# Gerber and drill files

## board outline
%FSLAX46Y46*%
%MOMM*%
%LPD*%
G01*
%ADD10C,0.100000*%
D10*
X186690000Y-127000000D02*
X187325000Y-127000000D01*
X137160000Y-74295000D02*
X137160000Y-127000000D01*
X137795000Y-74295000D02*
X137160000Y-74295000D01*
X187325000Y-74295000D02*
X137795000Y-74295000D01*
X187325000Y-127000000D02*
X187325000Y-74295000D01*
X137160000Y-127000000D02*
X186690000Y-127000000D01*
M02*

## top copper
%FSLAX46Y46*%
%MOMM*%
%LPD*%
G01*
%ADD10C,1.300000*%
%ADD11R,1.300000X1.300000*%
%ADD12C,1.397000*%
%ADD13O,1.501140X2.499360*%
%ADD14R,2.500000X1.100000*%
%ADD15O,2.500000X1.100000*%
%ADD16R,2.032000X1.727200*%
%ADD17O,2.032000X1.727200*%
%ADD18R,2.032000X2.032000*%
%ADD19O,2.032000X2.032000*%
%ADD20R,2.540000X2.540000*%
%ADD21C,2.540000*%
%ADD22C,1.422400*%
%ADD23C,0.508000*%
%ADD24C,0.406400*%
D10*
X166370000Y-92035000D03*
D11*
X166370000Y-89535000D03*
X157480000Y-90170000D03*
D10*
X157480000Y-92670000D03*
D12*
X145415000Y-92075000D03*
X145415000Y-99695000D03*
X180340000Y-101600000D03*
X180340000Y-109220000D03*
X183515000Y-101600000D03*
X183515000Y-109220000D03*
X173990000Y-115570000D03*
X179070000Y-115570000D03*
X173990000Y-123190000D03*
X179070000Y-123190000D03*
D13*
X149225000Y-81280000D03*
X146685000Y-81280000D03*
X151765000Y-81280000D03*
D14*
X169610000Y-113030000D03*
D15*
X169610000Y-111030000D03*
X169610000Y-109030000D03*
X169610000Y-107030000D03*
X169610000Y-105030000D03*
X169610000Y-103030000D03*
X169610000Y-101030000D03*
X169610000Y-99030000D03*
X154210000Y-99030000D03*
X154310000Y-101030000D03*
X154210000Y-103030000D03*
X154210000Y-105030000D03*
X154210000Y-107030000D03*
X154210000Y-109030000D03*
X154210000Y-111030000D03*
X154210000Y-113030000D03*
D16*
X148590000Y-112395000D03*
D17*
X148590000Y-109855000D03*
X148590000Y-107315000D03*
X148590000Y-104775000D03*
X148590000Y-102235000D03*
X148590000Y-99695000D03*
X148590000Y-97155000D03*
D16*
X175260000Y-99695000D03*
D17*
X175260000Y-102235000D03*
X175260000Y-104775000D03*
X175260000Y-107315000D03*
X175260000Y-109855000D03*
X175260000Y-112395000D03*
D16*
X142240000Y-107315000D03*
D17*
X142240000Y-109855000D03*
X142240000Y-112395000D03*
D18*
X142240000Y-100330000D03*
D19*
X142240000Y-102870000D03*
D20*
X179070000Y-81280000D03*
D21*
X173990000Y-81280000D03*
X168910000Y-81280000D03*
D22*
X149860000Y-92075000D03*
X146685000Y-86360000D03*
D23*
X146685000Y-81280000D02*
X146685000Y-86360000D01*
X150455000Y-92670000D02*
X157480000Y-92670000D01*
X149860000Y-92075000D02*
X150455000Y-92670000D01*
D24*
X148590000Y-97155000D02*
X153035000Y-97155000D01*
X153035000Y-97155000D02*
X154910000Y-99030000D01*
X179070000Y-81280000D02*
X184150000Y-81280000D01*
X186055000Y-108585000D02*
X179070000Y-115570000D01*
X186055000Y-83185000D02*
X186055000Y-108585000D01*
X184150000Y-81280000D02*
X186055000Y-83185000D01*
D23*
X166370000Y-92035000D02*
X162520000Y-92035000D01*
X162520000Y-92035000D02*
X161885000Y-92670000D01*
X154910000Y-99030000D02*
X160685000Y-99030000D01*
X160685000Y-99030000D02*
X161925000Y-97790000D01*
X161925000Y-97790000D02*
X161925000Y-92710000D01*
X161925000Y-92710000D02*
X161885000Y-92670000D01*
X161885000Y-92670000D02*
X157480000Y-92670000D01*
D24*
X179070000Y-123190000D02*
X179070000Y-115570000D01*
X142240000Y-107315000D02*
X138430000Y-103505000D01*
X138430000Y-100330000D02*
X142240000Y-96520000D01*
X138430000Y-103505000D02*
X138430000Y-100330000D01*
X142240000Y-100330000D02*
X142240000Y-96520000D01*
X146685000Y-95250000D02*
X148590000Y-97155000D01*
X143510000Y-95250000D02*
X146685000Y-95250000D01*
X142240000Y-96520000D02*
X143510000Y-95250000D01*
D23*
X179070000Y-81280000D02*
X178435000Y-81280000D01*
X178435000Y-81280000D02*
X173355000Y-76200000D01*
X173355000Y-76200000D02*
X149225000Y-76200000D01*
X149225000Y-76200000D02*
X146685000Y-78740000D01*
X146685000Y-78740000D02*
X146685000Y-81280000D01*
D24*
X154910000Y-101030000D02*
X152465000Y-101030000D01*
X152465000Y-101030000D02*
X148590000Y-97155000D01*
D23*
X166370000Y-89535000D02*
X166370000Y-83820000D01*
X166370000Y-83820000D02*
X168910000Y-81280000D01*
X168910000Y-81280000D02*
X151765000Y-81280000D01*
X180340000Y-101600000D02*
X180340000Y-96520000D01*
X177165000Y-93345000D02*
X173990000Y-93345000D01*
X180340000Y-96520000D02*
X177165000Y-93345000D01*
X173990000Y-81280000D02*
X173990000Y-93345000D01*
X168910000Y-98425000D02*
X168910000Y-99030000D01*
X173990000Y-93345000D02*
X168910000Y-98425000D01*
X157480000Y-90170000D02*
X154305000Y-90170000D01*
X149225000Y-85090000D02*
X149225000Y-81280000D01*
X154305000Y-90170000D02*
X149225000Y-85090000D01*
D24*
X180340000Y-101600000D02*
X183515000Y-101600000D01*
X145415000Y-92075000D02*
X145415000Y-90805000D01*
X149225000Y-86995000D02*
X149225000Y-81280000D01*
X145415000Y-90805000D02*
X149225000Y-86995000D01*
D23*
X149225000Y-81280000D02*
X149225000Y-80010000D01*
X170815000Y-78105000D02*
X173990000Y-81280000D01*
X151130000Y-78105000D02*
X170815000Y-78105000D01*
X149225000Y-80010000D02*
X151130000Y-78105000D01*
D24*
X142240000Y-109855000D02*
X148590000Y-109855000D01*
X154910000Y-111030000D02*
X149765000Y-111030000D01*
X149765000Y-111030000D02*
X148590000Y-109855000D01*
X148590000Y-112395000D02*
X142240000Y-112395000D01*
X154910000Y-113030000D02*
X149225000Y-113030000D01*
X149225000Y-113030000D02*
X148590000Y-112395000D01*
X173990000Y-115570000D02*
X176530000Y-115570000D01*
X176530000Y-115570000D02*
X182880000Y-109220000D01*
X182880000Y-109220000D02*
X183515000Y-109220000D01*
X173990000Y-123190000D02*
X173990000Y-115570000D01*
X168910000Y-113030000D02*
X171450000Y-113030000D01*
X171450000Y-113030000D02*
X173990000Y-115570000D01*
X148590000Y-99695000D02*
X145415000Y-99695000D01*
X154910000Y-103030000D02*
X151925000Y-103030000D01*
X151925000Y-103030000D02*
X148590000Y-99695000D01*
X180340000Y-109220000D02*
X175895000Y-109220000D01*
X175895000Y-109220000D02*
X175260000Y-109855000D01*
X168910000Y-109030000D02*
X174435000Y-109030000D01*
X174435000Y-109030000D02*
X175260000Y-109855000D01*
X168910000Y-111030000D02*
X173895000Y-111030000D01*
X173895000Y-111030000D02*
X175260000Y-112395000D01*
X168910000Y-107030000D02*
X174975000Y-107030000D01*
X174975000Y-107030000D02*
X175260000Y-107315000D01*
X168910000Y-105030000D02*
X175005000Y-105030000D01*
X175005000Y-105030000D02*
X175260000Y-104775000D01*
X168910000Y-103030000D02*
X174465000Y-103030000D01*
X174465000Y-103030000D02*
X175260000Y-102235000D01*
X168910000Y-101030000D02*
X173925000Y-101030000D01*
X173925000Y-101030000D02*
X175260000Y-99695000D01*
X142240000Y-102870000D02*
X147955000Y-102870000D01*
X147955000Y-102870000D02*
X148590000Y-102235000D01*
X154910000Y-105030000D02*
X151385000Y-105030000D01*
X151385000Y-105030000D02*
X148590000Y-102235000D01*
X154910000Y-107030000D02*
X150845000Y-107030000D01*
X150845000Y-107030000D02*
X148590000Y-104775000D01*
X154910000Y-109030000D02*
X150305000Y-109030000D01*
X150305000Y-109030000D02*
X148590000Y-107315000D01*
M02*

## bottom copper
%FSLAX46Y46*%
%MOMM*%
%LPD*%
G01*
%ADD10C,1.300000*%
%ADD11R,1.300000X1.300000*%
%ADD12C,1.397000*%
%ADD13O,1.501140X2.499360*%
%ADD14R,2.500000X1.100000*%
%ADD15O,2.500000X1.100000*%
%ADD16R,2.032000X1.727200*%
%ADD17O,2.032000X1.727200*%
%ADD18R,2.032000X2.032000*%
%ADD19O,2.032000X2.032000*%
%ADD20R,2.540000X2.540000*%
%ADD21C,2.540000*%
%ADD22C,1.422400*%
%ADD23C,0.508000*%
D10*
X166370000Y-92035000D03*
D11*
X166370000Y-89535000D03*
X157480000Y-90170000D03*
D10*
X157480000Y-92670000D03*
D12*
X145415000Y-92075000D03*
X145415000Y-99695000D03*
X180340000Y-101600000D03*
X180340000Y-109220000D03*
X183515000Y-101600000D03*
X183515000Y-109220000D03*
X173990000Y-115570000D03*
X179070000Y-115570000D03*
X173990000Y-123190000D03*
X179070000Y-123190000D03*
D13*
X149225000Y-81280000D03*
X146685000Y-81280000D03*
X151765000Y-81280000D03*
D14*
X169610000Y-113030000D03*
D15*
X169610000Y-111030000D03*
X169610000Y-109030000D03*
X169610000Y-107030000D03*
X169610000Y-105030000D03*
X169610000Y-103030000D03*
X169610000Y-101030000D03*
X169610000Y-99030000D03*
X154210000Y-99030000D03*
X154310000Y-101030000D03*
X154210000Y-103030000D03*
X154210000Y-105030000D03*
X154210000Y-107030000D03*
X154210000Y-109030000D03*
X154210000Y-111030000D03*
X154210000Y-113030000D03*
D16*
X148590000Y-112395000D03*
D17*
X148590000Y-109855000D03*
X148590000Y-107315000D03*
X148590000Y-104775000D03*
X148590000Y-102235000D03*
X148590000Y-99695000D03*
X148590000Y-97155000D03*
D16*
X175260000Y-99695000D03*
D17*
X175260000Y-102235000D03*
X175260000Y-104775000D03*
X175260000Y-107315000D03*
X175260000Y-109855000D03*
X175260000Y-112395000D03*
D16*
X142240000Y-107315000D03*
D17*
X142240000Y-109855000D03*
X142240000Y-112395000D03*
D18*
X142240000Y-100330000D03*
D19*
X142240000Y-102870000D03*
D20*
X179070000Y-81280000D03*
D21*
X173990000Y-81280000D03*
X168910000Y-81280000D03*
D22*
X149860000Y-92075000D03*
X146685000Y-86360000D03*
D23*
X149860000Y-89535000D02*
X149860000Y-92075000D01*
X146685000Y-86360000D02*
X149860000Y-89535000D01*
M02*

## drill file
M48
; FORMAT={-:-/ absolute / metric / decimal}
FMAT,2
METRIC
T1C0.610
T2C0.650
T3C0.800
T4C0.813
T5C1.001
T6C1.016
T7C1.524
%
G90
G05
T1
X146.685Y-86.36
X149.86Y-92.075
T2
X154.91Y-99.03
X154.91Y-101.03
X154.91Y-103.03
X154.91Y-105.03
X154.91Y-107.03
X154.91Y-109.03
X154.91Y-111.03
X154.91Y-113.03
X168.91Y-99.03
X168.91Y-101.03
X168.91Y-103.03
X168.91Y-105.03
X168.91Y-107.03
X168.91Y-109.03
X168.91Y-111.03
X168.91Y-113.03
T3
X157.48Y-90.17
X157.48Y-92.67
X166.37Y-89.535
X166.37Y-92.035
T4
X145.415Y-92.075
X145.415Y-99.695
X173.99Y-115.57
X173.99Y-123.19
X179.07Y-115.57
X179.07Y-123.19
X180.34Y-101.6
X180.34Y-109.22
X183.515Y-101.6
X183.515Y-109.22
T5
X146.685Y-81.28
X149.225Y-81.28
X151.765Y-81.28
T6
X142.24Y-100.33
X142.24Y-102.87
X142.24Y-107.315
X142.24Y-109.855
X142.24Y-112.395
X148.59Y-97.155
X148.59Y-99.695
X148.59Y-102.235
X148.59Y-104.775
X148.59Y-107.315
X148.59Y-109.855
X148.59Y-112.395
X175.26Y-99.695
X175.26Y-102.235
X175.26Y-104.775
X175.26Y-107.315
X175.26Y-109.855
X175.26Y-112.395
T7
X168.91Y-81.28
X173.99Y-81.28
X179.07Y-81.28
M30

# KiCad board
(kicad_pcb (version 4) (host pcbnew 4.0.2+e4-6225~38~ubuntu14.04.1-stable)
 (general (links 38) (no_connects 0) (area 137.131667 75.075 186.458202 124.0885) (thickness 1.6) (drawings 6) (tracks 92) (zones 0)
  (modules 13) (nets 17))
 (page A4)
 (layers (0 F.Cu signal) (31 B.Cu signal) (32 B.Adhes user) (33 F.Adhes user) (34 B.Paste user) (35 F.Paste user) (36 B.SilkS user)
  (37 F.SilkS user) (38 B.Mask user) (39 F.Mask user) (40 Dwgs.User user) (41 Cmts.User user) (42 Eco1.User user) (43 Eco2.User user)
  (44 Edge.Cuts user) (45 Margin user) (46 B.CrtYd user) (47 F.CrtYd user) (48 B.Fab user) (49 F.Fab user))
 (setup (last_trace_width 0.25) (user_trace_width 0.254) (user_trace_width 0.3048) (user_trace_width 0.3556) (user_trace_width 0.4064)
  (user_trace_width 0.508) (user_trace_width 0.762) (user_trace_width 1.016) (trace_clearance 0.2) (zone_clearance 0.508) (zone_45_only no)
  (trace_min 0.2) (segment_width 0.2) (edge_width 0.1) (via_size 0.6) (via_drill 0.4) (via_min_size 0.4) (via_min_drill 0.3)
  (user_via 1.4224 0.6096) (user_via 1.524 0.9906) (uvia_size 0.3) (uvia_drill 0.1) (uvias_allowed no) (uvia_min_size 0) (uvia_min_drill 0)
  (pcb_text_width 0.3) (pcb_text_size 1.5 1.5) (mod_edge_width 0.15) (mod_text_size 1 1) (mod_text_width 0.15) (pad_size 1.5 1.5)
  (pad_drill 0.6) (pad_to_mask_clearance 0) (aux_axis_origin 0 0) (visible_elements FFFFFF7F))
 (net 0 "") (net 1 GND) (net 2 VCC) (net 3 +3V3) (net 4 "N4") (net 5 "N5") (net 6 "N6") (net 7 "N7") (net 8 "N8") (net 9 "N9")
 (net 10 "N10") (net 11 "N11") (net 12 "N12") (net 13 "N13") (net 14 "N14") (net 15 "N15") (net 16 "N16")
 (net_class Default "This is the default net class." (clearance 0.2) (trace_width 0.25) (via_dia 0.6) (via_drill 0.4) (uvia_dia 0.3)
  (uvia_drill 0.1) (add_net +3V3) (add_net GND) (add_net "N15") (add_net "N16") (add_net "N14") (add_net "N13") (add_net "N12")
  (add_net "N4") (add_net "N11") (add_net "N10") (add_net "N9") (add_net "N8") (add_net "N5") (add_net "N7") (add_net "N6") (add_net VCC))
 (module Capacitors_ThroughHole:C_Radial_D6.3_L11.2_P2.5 (layer F.Cu) (at 166.37 89.535 270)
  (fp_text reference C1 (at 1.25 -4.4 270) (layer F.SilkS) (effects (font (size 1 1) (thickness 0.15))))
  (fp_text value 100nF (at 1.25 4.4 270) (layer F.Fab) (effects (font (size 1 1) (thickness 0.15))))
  (pad 2 thru_hole circle (at 2.5 0 270) (size 1.3 1.3) (drill 0.8) (layers *.Cu *.Mask F.SilkS) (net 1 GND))
  (pad 1 thru_hole rect (at 0 0 270) (size 1.3 1.3) (drill 0.8) (layers *.Cu *.Mask F.SilkS) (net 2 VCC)))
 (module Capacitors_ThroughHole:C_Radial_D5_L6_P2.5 (layer F.Cu) (at 157.48 90.17 270)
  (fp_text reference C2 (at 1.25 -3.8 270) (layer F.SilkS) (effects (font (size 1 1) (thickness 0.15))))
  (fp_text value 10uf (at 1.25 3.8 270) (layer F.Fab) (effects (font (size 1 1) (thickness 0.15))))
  (pad 1 thru_hole rect (at 0 0 270) (size 1.3 1.3) (drill 0.8) (layers *.Cu *.Mask F.SilkS) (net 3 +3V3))
  (pad 2 thru_hole circle (at 2.5 0 270) (size 1.3 1.3) (drill 0.8) (layers *.Cu *.Mask F.SilkS) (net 1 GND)))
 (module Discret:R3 (layer F.Cu) (at 145.415 95.885 270)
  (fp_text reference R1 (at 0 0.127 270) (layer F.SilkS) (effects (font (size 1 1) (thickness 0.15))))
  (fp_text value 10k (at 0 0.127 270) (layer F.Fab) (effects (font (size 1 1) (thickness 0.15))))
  (pad 1 thru_hole circle (at -3.81 0 270) (size 1.397 1.397) (drill 0.8128) (layers *.Cu *.Mask F.SilkS) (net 3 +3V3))
  (pad 2 thru_hole circle (at 3.81 0 270) (size 1.397 1.397) (drill 0.8128) (layers *.Cu *.Mask F.SilkS) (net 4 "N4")))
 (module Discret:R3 (layer F.Cu) (at 180.34 105.41 270)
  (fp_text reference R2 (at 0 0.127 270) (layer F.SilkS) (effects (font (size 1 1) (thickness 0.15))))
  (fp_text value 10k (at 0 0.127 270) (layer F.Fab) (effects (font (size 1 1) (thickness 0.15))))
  (pad 1 thru_hole circle (at -3.81 0 270) (size 1.397 1.397) (drill 0.8128) (layers *.Cu *.Mask F.SilkS) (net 3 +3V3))
  (pad 2 thru_hole circle (at 3.81 0 270) (size 1.397 1.397) (drill 0.8128) (layers *.Cu *.Mask F.SilkS) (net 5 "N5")))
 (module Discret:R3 (layer F.Cu) (at 183.515 105.41 270)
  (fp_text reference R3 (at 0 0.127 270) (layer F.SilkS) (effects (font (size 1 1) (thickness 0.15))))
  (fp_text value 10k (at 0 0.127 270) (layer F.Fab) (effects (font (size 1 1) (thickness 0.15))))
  (pad 1 thru_hole circle (at -3.81 0 270) (size 1.397 1.397) (drill 0.8128) (layers *.Cu *.Mask F.SilkS) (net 3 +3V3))
  (pad 2 thru_hole circle (at 3.81 0 270) (size 1.397 1.397) (drill 0.8128) (layers *.Cu *.Mask F.SilkS) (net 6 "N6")))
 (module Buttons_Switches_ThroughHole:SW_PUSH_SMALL (layer F.Cu) (at 176.53 119.38 90)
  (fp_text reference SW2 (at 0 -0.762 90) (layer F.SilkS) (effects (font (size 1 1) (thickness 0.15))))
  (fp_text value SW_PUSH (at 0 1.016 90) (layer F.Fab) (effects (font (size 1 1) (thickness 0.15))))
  (pad 1 thru_hole circle (at 3.81 -2.54 90) (size 1.397 1.397) (drill 0.8128) (layers *.Cu *.Mask F.SilkS) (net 6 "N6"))
  (pad 2 thru_hole circle (at 3.81 2.54 90) (size 1.397 1.397) (drill 0.8128) (layers *.Cu *.Mask F.SilkS) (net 1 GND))
  (pad 1 thru_hole circle (at -3.81 -2.54 90) (size 1.397 1.397) (drill 0.8128) (layers *.Cu *.Mask F.SilkS) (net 6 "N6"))
  (pad 2 thru_hole circle (at -3.81 2.54 90) (size 1.397 1.397) (drill 0.8128) (layers *.Cu *.Mask F.SilkS) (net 1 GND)))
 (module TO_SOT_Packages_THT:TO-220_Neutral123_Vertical (layer F.Cu) (at 149.225 81.28)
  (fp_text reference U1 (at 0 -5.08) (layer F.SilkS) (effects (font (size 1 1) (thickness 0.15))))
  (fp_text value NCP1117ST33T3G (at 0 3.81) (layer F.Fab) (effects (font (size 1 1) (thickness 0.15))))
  (pad 2 thru_hole oval (at 0 0 90) (size 2.49936 1.50114) (drill 1.00076) (layers *.Cu *.Mask F.SilkS) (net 3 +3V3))
  (pad 1 thru_hole oval (at -2.54 0 90) (size 2.49936 1.50114) (drill 1.00076) (layers *.Cu *.Mask F.SilkS) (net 1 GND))
  (pad 3 thru_hole oval (at 2.54 0 90) (size 2.49936 1.50114) (drill 1.00076) (layers *.Cu *.Mask F.SilkS) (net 2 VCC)))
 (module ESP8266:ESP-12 (layer F.Cu) (at 168.91 113.03 180)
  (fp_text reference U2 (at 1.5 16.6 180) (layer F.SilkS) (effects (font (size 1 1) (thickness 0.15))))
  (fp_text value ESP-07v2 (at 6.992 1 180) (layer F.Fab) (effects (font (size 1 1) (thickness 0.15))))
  (pad 1 thru_hole rect (at 0 0 180) (size 2.5 1.1) (drill 0.65 (offset -0.7 0)) (layers *.Cu *.Mask F.SilkS) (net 6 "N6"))
  (pad 2 thru_hole oval (at 0 2 180) (size 2.5 1.1) (drill 0.65 (offset -0.7 0)) (layers *.Cu *.Mask F.SilkS) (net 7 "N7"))
  (pad 3 thru_hole oval (at 0 4 180) (size 2.5 1.1) (drill 0.65 (offset -0.7 0)) (layers *.Cu *.Mask F.SilkS) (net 5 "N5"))
  (pad 4 thru_hole oval (at 0 6 180) (size 2.5 1.1) (drill 0.65 (offset -0.7 0)) (layers *.Cu *.Mask F.SilkS) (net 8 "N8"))
  (pad 5 thru_hole oval (at 0 8 180) (size 2.5 1.1) (drill 0.65 (offset -0.7 0)) (layers *.Cu *.Mask F.SilkS) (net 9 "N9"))
  (pad 6 thru_hole oval (at 0 10 180) (size 2.5 1.1) (drill 0.65 (offset -0.7 0)) (layers *.Cu *.Mask F.SilkS) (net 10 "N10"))
  (pad 7 thru_hole oval (at 0 12 180) (size 2.5 1.1) (drill 0.65 (offset -0.7 0)) (layers *.Cu *.Mask F.SilkS) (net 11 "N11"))
  (pad 8 thru_hole oval (at 0 14 180) (size 2.5 1.1) (drill 0.65 (offset -0.7 0)) (layers *.Cu *.Mask F.SilkS) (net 3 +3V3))
  (pad 9 thru_hole oval (at 14 14 180) (size 2.5 1.1) (drill 0.65 (offset 0.7 0)) (layers *.Cu *.Mask F.SilkS) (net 1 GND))
  (pad 10 thru_hole oval (at 14 12 180) (size 2.5 1.1) (drill 0.65 (offset 0.6 0)) (layers *.Cu *.Mask F.SilkS) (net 1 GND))
  (pad 11 thru_hole oval (at 14 10 180) (size 2.5 1.1) (drill 0.65 (offset 0.7 0)) (layers *.Cu *.Mask F.SilkS) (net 4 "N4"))
  (pad 12 thru_hole oval (at 14 8 180) (size 2.5 1.1) (drill 0.65 (offset 0.7 0)) (layers *.Cu *.Mask F.SilkS) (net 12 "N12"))
  (pad 13 thru_hole oval (at 14 6 180) (size 2.5 1.1) (drill 0.65 (offset 0.7 0)) (layers *.Cu *.Mask F.SilkS) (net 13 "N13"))
  (pad 14 thru_hole oval (at 14 4 180) (size 2.5 1.1) (drill 0.65 (offset 0.7 0)) (layers *.Cu *.Mask F.SilkS) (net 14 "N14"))
  (pad 15 thru_hole oval (at 14 2 180) (size 2.5 1.1) (drill 0.65 (offset 0.7 0)) (layers *.Cu *.Mask F.SilkS) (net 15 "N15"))
  (pad 16 thru_hole oval (at 14 0 180) (size 2.5 1.1) (drill 0.65 (offset 0.7 0)) (layers *.Cu *.Mask F.SilkS) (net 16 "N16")))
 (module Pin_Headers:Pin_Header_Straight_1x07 (layer F.Cu) (at 148.59 112.395 180)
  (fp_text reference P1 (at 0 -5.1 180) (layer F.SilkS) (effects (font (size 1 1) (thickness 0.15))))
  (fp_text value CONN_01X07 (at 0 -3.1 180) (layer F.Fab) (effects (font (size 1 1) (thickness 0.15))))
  (pad 1 thru_hole rect (at 0 0 180) (size 2.032 1.7272) (drill 1.016) (layers *.Cu *.Mask F.SilkS) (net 16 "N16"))
  (pad 2 thru_hole oval (at 0 2.54 180) (size 2.032 1.7272) (drill 1.016) (layers *.Cu *.Mask F.SilkS) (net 15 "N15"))
  (pad 3 thru_hole oval (at 0 5.08 180) (size 2.032 1.7272) (drill 1.016) (layers *.Cu *.Mask F.SilkS) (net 14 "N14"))
  (pad 4 thru_hole oval (at 0 7.62 180) (size 2.032 1.7272) (drill 1.016) (layers *.Cu *.Mask F.SilkS) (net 13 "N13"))
  (pad 5 thru_hole oval (at 0 10.16 180) (size 2.032 1.7272) (drill 1.016) (layers *.Cu *.Mask F.SilkS) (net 12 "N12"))
  (pad 6 thru_hole oval (at 0 12.7 180) (size 2.032 1.7272) (drill 1.016) (layers *.Cu *.Mask F.SilkS) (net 4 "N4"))
  (pad 7 thru_hole oval (at 0 15.24 180) (size 2.032 1.7272) (drill 1.016) (layers *.Cu *.Mask F.SilkS) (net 1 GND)))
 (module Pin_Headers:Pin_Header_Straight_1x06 (layer F.Cu) (at 175.26 99.695)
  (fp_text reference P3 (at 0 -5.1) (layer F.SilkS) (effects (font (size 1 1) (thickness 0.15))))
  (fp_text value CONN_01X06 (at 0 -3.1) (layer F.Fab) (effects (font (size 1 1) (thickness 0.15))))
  (pad 1 thru_hole rect (at 0 0) (size 2.032 1.7272) (drill 1.016) (layers *.Cu *.Mask F.SilkS) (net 11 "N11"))
  (pad 2 thru_hole oval (at 0 2.54) (size 2.032 1.7272) (drill 1.016) (layers *.Cu *.Mask F.SilkS) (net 10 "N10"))
  (pad 3 thru_hole oval (at 0 5.08) (size 2.032 1.7272) (drill 1.016) (layers *.Cu *.Mask F.SilkS) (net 9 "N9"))
  (pad 4 thru_hole oval (at 0 7.62) (size 2.032 1.7272) (drill 1.016) (layers *.Cu *.Mask F.SilkS) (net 8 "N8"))
  (pad 5 thru_hole oval (at 0 10.16) (size 2.032 1.7272) (drill 1.016) (layers *.Cu *.Mask F.SilkS) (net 5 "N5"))
  (pad 6 thru_hole oval (at 0 12.7) (size 2.032 1.7272) (drill 1.016) (layers *.Cu *.Mask F.SilkS) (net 7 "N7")))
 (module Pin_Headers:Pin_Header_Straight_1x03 (layer F.Cu) (at 142.24 107.315)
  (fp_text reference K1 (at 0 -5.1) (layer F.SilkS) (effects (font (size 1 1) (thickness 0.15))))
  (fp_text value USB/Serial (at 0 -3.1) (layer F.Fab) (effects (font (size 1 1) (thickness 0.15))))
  (pad 1 thru_hole rect (at 0 0) (size 2.032 1.7272) (drill 1.016) (layers *.Cu *.Mask F.SilkS) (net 1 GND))
  (pad 2 thru_hole oval (at 0 2.54) (size 2.032 1.7272) (drill 1.016) (layers *.Cu *.Mask F.SilkS) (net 15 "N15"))
  (pad 3 thru_hole oval (at 0 5.08) (size 2.032 1.7272) (drill 1.016) (layers *.Cu *.Mask F.SilkS) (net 16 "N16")))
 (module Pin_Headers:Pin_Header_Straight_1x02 (layer F.Cu) (at 142.24 100.33)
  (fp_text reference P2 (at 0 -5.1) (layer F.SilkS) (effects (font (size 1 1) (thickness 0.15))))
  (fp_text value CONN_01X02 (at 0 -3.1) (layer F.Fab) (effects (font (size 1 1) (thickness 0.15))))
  (pad 1 thru_hole rect (at 0 0) (size 2.032 2.032) (drill 1.016) (layers *.Cu *.Mask F.SilkS) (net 1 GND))
  (pad 2 thru_hole oval (at 0 2.54) (size 2.032 2.032) (drill 1.016) (layers *.Cu *.Mask F.SilkS) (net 12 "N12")))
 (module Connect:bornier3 (layer F.Cu) (at 173.99 81.28 180)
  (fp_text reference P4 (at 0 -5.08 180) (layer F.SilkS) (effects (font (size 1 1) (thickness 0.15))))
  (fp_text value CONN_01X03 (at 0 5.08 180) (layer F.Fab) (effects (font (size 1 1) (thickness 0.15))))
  (pad 1 thru_hole rect (at -5.08 0 180) (size 2.54 2.54) (drill 1.524) (layers *.Cu *.Mask F.SilkS) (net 1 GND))
  (pad 2 thru_hole circle (at 0 0 180) (size 2.54 2.54) (drill 1.524) (layers *.Cu *.Mask F.SilkS) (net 3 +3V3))
  (pad 3 thru_hole circle (at 5.08 0 180) (size 2.54 2.54) (drill 1.524) (layers *.Cu *.Mask F.SilkS) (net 2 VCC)))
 (gr_line (start 186.69 127) (end 187.325 127) (angle 90) (layer Edge.Cuts) (width 0.1))
 (gr_line (start 137.16 74.295) (end 137.16 127) (angle 90) (layer Edge.Cuts) (width 0.1))
 (gr_line (start 137.795 74.295) (end 137.16 74.295) (angle 90) (layer Edge.Cuts) (width 0.1))
 (gr_line (start 187.325 74.295) (end 137.795 74.295) (angle 90) (layer Edge.Cuts) (width 0.1))
 (gr_line (start 187.325 127) (end 187.325 74.295) (angle 90) (layer Edge.Cuts) (width 0.1))
 (gr_line (start 137.16 127) (end 186.69 127) (angle 90) (layer Edge.Cuts) (width 0.1))
 (segment (start 146.685 81.28) (end 146.685 86.36) (width 0.508) (layer F.Cu) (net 1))
 (segment (start 150.455 92.67) (end 157.48 92.67) (width 0.508) (layer F.Cu) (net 1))
 (segment (start 149.86 92.075) (end 150.455 92.67) (width 0.508) (layer F.Cu) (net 1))
 (via (at 149.86 92.075) (size 1.4224) (drill 0.6096) (layers F.Cu B.Cu) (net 1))
 (segment (start 149.86 89.535) (end 149.86 92.075) (width 0.508) (layer B.Cu) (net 1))
 (segment (start 146.685 86.36) (end 149.86 89.535) (width 0.508) (layer B.Cu) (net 1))
 (via (at 146.685 86.36) (size 1.4224) (drill 0.6096) (layers F.Cu B.Cu) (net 1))
 (segment (start 148.59 97.155) (end 153.035 97.155) (width 0.4064) (layer F.Cu) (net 1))
 (segment (start 153.035 97.155) (end 154.91 99.03) (width 0.4064) (layer F.Cu) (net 1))
 (segment (start 179.07 81.28) (end 184.15 81.28) (width 0.4064) (layer F.Cu) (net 1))
 (segment (start 186.055 108.585) (end 179.07 115.57) (width 0.4064) (layer F.Cu) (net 1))
 (segment (start 186.055 83.185) (end 186.055 108.585) (width 0.4064) (layer F.Cu) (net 1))
 (segment (start 184.15 81.28) (end 186.055 83.185) (width 0.4064) (layer F.Cu) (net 1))
 (segment (start 166.37 92.035) (end 162.52 92.035) (width 0.508) (layer F.Cu) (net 1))
 (segment (start 162.52 92.035) (end 161.885 92.67) (width 0.508) (layer F.Cu) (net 1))
 (segment (start 154.91 99.03) (end 160.685 99.03) (width 0.508) (layer F.Cu) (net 1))
 (segment (start 160.685 99.03) (end 161.925 97.79) (width 0.508) (layer F.Cu) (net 1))
 (segment (start 161.925 97.79) (end 161.925 92.71) (width 0.508) (layer F.Cu) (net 1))
 (segment (start 161.925 92.71) (end 161.885 92.67) (width 0.508) (layer F.Cu) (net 1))
 (segment (start 161.885 92.67) (end 157.48 92.67) (width 0.508) (layer F.Cu) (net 1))
 (segment (start 179.07 123.19) (end 179.07 115.57) (width 0.4064) (layer F.Cu) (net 1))
 (segment (start 142.24 107.315) (end 138.43 103.505) (width 0.4064) (layer F.Cu) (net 1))
 (segment (start 138.43 100.33) (end 142.24 96.52) (width 0.4064) (layer F.Cu) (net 1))
 (segment (start 138.43 103.505) (end 138.43 100.33) (width 0.4064) (layer F.Cu) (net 1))
 (segment (start 142.24 100.33) (end 142.24 96.52) (width 0.4064) (layer F.Cu) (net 1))
 (segment (start 146.685 95.25) (end 148.59 97.155) (width 0.4064) (layer F.Cu) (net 1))
 (segment (start 143.51 95.25) (end 146.685 95.25) (width 0.4064) (layer F.Cu) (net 1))
 (segment (start 142.24 96.52) (end 143.51 95.25) (width 0.4064) (layer F.Cu) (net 1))
 (segment (start 179.07 81.28) (end 178.435 81.28) (width 0.508) (layer F.Cu) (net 1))
 (segment (start 178.435 81.28) (end 173.355 76.2) (width 0.508) (layer F.Cu) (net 1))
 (segment (start 173.355 76.2) (end 149.225 76.2) (width 0.508) (layer F.Cu) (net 1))
 (segment (start 149.225 76.2) (end 146.685 78.74) (width 0.508) (layer F.Cu) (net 1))
 (segment (start 146.685 78.74) (end 146.685 81.28) (width 0.508) (layer F.Cu) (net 1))
 (segment (start 154.91 101.03) (end 152.465 101.03) (width 0.4064) (layer F.Cu) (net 1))
 (segment (start 152.465 101.03) (end 148.59 97.155) (width 0.4064) (layer F.Cu) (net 1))
 (segment (start 166.37 89.535) (end 166.37 83.82) (width 0.508) (layer F.Cu) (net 2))
 (segment (start 166.37 83.82) (end 168.91 81.28) (width 0.508) (layer F.Cu) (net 2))
 (segment (start 168.91 81.28) (end 151.765 81.28) (width 0.508) (layer F.Cu) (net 2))
 (segment (start 180.34 101.6) (end 180.34 96.52) (width 0.508) (layer F.Cu) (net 3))
 (segment (start 177.165 93.345) (end 173.99 93.345) (width 0.508) (layer F.Cu) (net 3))
 (segment (start 180.34 96.52) (end 177.165 93.345) (width 0.508) (layer F.Cu) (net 3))
 (segment (start 173.99 81.28) (end 173.99 93.345) (width 0.508) (layer F.Cu) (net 3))
 (segment (start 168.91 98.425) (end 168.91 99.03) (width 0.508) (layer F.Cu) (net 3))
 (segment (start 173.99 93.345) (end 168.91 98.425) (width 0.508) (layer F.Cu) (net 3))
 (segment (start 157.48 90.17) (end 154.305 90.17) (width 0.508) (layer F.Cu) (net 3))
 (segment (start 149.225 85.09) (end 149.225 81.28) (width 0.508) (layer F.Cu) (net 3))
 (segment (start 154.305 90.17) (end 149.225 85.09) (width 0.508) (layer F.Cu) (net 3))
 (segment (start 180.34 101.6) (end 183.515 101.6) (width 0.4064) (layer F.Cu) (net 3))
 (segment (start 145.415 92.075) (end 145.415 90.805) (width 0.4064) (layer F.Cu) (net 3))
 (segment (start 149.225 86.995) (end 149.225 81.28) (width 0.4064) (layer F.Cu) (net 3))
 (segment (start 145.415 90.805) (end 149.225 86.995) (width 0.4064) (layer F.Cu) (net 3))
 (segment (start 149.225 81.28) (end 149.225 80.01) (width 0.508) (layer F.Cu) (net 3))
 (segment (start 170.815 78.105) (end 173.99 81.28) (width 0.508) (layer F.Cu) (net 3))
 (segment (start 151.13 78.105) (end 170.815 78.105) (width 0.508) (layer F.Cu) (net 3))
 (segment (start 149.225 80.01) (end 151.13 78.105) (width 0.508) (layer F.Cu) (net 3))
 (segment (start 142.24 109.855) (end 148.59 109.855) (width 0.4064) (layer F.Cu) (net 15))
 (segment (start 154.91 111.03) (end 149.765 111.03) (width 0.4064) (layer F.Cu) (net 15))
 (segment (start 149.765 111.03) (end 148.59 109.855) (width 0.4064) (layer F.Cu) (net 15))
 (segment (start 148.59 112.395) (end 142.24 112.395) (width 0.4064) (layer F.Cu) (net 16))
 (segment (start 154.91 113.03) (end 149.225 113.03) (width 0.4064) (layer F.Cu) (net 16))
 (segment (start 149.225 113.03) (end 148.59 112.395) (width 0.4064) (layer F.Cu) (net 16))
 (segment (start 173.99 115.57) (end 176.53 115.57) (width 0.4064) (layer F.Cu) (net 6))
 (segment (start 176.53 115.57) (end 182.88 109.22) (width 0.4064) (layer F.Cu) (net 6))
 (segment (start 182.88 109.22) (end 183.515 109.22) (width 0.4064) (layer F.Cu) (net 6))
 (segment (start 173.99 123.19) (end 173.99 115.57) (width 0.4064) (layer F.Cu) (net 6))
 (segment (start 168.91 113.03) (end 171.45 113.03) (width 0.4064) (layer F.Cu) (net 6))
 (segment (start 171.45 113.03) (end 173.99 115.57) (width 0.4064) (layer F.Cu) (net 6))
 (segment (start 148.59 99.695) (end 145.415 99.695) (width 0.4064) (layer F.Cu) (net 4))
 (segment (start 154.91 103.03) (end 151.925 103.03) (width 0.4064) (layer F.Cu) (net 4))
 (segment (start 151.925 103.03) (end 148.59 99.695) (width 0.4064) (layer F.Cu) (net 4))
 (segment (start 180.34 109.22) (end 175.895 109.22) (width 0.4064) (layer F.Cu) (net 5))
 (segment (start 175.895 109.22) (end 175.26 109.855) (width 0.4064) (layer F.Cu) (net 5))
 (segment (start 168.91 109.03) (end 174.435 109.03) (width 0.4064) (layer F.Cu) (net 5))
 (segment (start 174.435 109.03) (end 175.26 109.855) (width 0.4064) (layer F.Cu) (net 5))
 (segment (start 168.91 111.03) (end 173.895 111.03) (width 0.4064) (layer F.Cu) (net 7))
 (segment (start 173.895 111.03) (end 175.26 112.395) (width 0.4064) (layer F.Cu) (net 7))
 (segment (start 168.91 107.03) (end 174.975 107.03) (width 0.4064) (layer F.Cu) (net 8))
 (segment (start 174.975 107.03) (end 175.26 107.315) (width 0.4064) (layer F.Cu) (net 8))
 (segment (start 168.91 105.03) (end 175.005 105.03) (width 0.4064) (layer F.Cu) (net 9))
 (segment (start 175.005 105.03) (end 175.26 104.775) (width 0.4064) (layer F.Cu) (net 9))
 (segment (start 168.91 103.03) (end 174.465 103.03) (width 0.4064) (layer F.Cu) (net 10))
 (segment (start 174.465 103.03) (end 175.26 102.235) (width 0.4064) (layer F.Cu) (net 10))
 (segment (start 168.91 101.03) (end 173.925 101.03) (width 0.4064) (layer F.Cu) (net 11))
 (segment (start 173.925 101.03) (end 175.26 99.695) (width 0.4064) (layer F.Cu) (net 11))
 (segment (start 142.24 102.87) (end 147.955 102.87) (width 0.4064) (layer F.Cu) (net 12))
 (segment (start 147.955 102.87) (end 148.59 102.235) (width 0.4064) (layer F.Cu) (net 12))
 (segment (start 154.91 105.03) (end 151.385 105.03) (width 0.4064) (layer F.Cu) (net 12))
 (segment (start 151.385 105.03) (end 148.59 102.235) (width 0.4064) (layer F.Cu) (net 12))
 (segment (start 154.91 107.03) (end 150.845 107.03) (width 0.4064) (layer F.Cu) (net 13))
 (segment (start 150.845 107.03) (end 148.59 104.775) (width 0.4064) (layer F.Cu) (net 13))
 (segment (start 154.91 109.03) (end 150.305 109.03) (width 0.4064) (layer F.Cu) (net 14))
 (segment (start 150.305 109.03) (end 148.59 107.315) (width 0.4064) (layer F.Cu) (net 14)))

